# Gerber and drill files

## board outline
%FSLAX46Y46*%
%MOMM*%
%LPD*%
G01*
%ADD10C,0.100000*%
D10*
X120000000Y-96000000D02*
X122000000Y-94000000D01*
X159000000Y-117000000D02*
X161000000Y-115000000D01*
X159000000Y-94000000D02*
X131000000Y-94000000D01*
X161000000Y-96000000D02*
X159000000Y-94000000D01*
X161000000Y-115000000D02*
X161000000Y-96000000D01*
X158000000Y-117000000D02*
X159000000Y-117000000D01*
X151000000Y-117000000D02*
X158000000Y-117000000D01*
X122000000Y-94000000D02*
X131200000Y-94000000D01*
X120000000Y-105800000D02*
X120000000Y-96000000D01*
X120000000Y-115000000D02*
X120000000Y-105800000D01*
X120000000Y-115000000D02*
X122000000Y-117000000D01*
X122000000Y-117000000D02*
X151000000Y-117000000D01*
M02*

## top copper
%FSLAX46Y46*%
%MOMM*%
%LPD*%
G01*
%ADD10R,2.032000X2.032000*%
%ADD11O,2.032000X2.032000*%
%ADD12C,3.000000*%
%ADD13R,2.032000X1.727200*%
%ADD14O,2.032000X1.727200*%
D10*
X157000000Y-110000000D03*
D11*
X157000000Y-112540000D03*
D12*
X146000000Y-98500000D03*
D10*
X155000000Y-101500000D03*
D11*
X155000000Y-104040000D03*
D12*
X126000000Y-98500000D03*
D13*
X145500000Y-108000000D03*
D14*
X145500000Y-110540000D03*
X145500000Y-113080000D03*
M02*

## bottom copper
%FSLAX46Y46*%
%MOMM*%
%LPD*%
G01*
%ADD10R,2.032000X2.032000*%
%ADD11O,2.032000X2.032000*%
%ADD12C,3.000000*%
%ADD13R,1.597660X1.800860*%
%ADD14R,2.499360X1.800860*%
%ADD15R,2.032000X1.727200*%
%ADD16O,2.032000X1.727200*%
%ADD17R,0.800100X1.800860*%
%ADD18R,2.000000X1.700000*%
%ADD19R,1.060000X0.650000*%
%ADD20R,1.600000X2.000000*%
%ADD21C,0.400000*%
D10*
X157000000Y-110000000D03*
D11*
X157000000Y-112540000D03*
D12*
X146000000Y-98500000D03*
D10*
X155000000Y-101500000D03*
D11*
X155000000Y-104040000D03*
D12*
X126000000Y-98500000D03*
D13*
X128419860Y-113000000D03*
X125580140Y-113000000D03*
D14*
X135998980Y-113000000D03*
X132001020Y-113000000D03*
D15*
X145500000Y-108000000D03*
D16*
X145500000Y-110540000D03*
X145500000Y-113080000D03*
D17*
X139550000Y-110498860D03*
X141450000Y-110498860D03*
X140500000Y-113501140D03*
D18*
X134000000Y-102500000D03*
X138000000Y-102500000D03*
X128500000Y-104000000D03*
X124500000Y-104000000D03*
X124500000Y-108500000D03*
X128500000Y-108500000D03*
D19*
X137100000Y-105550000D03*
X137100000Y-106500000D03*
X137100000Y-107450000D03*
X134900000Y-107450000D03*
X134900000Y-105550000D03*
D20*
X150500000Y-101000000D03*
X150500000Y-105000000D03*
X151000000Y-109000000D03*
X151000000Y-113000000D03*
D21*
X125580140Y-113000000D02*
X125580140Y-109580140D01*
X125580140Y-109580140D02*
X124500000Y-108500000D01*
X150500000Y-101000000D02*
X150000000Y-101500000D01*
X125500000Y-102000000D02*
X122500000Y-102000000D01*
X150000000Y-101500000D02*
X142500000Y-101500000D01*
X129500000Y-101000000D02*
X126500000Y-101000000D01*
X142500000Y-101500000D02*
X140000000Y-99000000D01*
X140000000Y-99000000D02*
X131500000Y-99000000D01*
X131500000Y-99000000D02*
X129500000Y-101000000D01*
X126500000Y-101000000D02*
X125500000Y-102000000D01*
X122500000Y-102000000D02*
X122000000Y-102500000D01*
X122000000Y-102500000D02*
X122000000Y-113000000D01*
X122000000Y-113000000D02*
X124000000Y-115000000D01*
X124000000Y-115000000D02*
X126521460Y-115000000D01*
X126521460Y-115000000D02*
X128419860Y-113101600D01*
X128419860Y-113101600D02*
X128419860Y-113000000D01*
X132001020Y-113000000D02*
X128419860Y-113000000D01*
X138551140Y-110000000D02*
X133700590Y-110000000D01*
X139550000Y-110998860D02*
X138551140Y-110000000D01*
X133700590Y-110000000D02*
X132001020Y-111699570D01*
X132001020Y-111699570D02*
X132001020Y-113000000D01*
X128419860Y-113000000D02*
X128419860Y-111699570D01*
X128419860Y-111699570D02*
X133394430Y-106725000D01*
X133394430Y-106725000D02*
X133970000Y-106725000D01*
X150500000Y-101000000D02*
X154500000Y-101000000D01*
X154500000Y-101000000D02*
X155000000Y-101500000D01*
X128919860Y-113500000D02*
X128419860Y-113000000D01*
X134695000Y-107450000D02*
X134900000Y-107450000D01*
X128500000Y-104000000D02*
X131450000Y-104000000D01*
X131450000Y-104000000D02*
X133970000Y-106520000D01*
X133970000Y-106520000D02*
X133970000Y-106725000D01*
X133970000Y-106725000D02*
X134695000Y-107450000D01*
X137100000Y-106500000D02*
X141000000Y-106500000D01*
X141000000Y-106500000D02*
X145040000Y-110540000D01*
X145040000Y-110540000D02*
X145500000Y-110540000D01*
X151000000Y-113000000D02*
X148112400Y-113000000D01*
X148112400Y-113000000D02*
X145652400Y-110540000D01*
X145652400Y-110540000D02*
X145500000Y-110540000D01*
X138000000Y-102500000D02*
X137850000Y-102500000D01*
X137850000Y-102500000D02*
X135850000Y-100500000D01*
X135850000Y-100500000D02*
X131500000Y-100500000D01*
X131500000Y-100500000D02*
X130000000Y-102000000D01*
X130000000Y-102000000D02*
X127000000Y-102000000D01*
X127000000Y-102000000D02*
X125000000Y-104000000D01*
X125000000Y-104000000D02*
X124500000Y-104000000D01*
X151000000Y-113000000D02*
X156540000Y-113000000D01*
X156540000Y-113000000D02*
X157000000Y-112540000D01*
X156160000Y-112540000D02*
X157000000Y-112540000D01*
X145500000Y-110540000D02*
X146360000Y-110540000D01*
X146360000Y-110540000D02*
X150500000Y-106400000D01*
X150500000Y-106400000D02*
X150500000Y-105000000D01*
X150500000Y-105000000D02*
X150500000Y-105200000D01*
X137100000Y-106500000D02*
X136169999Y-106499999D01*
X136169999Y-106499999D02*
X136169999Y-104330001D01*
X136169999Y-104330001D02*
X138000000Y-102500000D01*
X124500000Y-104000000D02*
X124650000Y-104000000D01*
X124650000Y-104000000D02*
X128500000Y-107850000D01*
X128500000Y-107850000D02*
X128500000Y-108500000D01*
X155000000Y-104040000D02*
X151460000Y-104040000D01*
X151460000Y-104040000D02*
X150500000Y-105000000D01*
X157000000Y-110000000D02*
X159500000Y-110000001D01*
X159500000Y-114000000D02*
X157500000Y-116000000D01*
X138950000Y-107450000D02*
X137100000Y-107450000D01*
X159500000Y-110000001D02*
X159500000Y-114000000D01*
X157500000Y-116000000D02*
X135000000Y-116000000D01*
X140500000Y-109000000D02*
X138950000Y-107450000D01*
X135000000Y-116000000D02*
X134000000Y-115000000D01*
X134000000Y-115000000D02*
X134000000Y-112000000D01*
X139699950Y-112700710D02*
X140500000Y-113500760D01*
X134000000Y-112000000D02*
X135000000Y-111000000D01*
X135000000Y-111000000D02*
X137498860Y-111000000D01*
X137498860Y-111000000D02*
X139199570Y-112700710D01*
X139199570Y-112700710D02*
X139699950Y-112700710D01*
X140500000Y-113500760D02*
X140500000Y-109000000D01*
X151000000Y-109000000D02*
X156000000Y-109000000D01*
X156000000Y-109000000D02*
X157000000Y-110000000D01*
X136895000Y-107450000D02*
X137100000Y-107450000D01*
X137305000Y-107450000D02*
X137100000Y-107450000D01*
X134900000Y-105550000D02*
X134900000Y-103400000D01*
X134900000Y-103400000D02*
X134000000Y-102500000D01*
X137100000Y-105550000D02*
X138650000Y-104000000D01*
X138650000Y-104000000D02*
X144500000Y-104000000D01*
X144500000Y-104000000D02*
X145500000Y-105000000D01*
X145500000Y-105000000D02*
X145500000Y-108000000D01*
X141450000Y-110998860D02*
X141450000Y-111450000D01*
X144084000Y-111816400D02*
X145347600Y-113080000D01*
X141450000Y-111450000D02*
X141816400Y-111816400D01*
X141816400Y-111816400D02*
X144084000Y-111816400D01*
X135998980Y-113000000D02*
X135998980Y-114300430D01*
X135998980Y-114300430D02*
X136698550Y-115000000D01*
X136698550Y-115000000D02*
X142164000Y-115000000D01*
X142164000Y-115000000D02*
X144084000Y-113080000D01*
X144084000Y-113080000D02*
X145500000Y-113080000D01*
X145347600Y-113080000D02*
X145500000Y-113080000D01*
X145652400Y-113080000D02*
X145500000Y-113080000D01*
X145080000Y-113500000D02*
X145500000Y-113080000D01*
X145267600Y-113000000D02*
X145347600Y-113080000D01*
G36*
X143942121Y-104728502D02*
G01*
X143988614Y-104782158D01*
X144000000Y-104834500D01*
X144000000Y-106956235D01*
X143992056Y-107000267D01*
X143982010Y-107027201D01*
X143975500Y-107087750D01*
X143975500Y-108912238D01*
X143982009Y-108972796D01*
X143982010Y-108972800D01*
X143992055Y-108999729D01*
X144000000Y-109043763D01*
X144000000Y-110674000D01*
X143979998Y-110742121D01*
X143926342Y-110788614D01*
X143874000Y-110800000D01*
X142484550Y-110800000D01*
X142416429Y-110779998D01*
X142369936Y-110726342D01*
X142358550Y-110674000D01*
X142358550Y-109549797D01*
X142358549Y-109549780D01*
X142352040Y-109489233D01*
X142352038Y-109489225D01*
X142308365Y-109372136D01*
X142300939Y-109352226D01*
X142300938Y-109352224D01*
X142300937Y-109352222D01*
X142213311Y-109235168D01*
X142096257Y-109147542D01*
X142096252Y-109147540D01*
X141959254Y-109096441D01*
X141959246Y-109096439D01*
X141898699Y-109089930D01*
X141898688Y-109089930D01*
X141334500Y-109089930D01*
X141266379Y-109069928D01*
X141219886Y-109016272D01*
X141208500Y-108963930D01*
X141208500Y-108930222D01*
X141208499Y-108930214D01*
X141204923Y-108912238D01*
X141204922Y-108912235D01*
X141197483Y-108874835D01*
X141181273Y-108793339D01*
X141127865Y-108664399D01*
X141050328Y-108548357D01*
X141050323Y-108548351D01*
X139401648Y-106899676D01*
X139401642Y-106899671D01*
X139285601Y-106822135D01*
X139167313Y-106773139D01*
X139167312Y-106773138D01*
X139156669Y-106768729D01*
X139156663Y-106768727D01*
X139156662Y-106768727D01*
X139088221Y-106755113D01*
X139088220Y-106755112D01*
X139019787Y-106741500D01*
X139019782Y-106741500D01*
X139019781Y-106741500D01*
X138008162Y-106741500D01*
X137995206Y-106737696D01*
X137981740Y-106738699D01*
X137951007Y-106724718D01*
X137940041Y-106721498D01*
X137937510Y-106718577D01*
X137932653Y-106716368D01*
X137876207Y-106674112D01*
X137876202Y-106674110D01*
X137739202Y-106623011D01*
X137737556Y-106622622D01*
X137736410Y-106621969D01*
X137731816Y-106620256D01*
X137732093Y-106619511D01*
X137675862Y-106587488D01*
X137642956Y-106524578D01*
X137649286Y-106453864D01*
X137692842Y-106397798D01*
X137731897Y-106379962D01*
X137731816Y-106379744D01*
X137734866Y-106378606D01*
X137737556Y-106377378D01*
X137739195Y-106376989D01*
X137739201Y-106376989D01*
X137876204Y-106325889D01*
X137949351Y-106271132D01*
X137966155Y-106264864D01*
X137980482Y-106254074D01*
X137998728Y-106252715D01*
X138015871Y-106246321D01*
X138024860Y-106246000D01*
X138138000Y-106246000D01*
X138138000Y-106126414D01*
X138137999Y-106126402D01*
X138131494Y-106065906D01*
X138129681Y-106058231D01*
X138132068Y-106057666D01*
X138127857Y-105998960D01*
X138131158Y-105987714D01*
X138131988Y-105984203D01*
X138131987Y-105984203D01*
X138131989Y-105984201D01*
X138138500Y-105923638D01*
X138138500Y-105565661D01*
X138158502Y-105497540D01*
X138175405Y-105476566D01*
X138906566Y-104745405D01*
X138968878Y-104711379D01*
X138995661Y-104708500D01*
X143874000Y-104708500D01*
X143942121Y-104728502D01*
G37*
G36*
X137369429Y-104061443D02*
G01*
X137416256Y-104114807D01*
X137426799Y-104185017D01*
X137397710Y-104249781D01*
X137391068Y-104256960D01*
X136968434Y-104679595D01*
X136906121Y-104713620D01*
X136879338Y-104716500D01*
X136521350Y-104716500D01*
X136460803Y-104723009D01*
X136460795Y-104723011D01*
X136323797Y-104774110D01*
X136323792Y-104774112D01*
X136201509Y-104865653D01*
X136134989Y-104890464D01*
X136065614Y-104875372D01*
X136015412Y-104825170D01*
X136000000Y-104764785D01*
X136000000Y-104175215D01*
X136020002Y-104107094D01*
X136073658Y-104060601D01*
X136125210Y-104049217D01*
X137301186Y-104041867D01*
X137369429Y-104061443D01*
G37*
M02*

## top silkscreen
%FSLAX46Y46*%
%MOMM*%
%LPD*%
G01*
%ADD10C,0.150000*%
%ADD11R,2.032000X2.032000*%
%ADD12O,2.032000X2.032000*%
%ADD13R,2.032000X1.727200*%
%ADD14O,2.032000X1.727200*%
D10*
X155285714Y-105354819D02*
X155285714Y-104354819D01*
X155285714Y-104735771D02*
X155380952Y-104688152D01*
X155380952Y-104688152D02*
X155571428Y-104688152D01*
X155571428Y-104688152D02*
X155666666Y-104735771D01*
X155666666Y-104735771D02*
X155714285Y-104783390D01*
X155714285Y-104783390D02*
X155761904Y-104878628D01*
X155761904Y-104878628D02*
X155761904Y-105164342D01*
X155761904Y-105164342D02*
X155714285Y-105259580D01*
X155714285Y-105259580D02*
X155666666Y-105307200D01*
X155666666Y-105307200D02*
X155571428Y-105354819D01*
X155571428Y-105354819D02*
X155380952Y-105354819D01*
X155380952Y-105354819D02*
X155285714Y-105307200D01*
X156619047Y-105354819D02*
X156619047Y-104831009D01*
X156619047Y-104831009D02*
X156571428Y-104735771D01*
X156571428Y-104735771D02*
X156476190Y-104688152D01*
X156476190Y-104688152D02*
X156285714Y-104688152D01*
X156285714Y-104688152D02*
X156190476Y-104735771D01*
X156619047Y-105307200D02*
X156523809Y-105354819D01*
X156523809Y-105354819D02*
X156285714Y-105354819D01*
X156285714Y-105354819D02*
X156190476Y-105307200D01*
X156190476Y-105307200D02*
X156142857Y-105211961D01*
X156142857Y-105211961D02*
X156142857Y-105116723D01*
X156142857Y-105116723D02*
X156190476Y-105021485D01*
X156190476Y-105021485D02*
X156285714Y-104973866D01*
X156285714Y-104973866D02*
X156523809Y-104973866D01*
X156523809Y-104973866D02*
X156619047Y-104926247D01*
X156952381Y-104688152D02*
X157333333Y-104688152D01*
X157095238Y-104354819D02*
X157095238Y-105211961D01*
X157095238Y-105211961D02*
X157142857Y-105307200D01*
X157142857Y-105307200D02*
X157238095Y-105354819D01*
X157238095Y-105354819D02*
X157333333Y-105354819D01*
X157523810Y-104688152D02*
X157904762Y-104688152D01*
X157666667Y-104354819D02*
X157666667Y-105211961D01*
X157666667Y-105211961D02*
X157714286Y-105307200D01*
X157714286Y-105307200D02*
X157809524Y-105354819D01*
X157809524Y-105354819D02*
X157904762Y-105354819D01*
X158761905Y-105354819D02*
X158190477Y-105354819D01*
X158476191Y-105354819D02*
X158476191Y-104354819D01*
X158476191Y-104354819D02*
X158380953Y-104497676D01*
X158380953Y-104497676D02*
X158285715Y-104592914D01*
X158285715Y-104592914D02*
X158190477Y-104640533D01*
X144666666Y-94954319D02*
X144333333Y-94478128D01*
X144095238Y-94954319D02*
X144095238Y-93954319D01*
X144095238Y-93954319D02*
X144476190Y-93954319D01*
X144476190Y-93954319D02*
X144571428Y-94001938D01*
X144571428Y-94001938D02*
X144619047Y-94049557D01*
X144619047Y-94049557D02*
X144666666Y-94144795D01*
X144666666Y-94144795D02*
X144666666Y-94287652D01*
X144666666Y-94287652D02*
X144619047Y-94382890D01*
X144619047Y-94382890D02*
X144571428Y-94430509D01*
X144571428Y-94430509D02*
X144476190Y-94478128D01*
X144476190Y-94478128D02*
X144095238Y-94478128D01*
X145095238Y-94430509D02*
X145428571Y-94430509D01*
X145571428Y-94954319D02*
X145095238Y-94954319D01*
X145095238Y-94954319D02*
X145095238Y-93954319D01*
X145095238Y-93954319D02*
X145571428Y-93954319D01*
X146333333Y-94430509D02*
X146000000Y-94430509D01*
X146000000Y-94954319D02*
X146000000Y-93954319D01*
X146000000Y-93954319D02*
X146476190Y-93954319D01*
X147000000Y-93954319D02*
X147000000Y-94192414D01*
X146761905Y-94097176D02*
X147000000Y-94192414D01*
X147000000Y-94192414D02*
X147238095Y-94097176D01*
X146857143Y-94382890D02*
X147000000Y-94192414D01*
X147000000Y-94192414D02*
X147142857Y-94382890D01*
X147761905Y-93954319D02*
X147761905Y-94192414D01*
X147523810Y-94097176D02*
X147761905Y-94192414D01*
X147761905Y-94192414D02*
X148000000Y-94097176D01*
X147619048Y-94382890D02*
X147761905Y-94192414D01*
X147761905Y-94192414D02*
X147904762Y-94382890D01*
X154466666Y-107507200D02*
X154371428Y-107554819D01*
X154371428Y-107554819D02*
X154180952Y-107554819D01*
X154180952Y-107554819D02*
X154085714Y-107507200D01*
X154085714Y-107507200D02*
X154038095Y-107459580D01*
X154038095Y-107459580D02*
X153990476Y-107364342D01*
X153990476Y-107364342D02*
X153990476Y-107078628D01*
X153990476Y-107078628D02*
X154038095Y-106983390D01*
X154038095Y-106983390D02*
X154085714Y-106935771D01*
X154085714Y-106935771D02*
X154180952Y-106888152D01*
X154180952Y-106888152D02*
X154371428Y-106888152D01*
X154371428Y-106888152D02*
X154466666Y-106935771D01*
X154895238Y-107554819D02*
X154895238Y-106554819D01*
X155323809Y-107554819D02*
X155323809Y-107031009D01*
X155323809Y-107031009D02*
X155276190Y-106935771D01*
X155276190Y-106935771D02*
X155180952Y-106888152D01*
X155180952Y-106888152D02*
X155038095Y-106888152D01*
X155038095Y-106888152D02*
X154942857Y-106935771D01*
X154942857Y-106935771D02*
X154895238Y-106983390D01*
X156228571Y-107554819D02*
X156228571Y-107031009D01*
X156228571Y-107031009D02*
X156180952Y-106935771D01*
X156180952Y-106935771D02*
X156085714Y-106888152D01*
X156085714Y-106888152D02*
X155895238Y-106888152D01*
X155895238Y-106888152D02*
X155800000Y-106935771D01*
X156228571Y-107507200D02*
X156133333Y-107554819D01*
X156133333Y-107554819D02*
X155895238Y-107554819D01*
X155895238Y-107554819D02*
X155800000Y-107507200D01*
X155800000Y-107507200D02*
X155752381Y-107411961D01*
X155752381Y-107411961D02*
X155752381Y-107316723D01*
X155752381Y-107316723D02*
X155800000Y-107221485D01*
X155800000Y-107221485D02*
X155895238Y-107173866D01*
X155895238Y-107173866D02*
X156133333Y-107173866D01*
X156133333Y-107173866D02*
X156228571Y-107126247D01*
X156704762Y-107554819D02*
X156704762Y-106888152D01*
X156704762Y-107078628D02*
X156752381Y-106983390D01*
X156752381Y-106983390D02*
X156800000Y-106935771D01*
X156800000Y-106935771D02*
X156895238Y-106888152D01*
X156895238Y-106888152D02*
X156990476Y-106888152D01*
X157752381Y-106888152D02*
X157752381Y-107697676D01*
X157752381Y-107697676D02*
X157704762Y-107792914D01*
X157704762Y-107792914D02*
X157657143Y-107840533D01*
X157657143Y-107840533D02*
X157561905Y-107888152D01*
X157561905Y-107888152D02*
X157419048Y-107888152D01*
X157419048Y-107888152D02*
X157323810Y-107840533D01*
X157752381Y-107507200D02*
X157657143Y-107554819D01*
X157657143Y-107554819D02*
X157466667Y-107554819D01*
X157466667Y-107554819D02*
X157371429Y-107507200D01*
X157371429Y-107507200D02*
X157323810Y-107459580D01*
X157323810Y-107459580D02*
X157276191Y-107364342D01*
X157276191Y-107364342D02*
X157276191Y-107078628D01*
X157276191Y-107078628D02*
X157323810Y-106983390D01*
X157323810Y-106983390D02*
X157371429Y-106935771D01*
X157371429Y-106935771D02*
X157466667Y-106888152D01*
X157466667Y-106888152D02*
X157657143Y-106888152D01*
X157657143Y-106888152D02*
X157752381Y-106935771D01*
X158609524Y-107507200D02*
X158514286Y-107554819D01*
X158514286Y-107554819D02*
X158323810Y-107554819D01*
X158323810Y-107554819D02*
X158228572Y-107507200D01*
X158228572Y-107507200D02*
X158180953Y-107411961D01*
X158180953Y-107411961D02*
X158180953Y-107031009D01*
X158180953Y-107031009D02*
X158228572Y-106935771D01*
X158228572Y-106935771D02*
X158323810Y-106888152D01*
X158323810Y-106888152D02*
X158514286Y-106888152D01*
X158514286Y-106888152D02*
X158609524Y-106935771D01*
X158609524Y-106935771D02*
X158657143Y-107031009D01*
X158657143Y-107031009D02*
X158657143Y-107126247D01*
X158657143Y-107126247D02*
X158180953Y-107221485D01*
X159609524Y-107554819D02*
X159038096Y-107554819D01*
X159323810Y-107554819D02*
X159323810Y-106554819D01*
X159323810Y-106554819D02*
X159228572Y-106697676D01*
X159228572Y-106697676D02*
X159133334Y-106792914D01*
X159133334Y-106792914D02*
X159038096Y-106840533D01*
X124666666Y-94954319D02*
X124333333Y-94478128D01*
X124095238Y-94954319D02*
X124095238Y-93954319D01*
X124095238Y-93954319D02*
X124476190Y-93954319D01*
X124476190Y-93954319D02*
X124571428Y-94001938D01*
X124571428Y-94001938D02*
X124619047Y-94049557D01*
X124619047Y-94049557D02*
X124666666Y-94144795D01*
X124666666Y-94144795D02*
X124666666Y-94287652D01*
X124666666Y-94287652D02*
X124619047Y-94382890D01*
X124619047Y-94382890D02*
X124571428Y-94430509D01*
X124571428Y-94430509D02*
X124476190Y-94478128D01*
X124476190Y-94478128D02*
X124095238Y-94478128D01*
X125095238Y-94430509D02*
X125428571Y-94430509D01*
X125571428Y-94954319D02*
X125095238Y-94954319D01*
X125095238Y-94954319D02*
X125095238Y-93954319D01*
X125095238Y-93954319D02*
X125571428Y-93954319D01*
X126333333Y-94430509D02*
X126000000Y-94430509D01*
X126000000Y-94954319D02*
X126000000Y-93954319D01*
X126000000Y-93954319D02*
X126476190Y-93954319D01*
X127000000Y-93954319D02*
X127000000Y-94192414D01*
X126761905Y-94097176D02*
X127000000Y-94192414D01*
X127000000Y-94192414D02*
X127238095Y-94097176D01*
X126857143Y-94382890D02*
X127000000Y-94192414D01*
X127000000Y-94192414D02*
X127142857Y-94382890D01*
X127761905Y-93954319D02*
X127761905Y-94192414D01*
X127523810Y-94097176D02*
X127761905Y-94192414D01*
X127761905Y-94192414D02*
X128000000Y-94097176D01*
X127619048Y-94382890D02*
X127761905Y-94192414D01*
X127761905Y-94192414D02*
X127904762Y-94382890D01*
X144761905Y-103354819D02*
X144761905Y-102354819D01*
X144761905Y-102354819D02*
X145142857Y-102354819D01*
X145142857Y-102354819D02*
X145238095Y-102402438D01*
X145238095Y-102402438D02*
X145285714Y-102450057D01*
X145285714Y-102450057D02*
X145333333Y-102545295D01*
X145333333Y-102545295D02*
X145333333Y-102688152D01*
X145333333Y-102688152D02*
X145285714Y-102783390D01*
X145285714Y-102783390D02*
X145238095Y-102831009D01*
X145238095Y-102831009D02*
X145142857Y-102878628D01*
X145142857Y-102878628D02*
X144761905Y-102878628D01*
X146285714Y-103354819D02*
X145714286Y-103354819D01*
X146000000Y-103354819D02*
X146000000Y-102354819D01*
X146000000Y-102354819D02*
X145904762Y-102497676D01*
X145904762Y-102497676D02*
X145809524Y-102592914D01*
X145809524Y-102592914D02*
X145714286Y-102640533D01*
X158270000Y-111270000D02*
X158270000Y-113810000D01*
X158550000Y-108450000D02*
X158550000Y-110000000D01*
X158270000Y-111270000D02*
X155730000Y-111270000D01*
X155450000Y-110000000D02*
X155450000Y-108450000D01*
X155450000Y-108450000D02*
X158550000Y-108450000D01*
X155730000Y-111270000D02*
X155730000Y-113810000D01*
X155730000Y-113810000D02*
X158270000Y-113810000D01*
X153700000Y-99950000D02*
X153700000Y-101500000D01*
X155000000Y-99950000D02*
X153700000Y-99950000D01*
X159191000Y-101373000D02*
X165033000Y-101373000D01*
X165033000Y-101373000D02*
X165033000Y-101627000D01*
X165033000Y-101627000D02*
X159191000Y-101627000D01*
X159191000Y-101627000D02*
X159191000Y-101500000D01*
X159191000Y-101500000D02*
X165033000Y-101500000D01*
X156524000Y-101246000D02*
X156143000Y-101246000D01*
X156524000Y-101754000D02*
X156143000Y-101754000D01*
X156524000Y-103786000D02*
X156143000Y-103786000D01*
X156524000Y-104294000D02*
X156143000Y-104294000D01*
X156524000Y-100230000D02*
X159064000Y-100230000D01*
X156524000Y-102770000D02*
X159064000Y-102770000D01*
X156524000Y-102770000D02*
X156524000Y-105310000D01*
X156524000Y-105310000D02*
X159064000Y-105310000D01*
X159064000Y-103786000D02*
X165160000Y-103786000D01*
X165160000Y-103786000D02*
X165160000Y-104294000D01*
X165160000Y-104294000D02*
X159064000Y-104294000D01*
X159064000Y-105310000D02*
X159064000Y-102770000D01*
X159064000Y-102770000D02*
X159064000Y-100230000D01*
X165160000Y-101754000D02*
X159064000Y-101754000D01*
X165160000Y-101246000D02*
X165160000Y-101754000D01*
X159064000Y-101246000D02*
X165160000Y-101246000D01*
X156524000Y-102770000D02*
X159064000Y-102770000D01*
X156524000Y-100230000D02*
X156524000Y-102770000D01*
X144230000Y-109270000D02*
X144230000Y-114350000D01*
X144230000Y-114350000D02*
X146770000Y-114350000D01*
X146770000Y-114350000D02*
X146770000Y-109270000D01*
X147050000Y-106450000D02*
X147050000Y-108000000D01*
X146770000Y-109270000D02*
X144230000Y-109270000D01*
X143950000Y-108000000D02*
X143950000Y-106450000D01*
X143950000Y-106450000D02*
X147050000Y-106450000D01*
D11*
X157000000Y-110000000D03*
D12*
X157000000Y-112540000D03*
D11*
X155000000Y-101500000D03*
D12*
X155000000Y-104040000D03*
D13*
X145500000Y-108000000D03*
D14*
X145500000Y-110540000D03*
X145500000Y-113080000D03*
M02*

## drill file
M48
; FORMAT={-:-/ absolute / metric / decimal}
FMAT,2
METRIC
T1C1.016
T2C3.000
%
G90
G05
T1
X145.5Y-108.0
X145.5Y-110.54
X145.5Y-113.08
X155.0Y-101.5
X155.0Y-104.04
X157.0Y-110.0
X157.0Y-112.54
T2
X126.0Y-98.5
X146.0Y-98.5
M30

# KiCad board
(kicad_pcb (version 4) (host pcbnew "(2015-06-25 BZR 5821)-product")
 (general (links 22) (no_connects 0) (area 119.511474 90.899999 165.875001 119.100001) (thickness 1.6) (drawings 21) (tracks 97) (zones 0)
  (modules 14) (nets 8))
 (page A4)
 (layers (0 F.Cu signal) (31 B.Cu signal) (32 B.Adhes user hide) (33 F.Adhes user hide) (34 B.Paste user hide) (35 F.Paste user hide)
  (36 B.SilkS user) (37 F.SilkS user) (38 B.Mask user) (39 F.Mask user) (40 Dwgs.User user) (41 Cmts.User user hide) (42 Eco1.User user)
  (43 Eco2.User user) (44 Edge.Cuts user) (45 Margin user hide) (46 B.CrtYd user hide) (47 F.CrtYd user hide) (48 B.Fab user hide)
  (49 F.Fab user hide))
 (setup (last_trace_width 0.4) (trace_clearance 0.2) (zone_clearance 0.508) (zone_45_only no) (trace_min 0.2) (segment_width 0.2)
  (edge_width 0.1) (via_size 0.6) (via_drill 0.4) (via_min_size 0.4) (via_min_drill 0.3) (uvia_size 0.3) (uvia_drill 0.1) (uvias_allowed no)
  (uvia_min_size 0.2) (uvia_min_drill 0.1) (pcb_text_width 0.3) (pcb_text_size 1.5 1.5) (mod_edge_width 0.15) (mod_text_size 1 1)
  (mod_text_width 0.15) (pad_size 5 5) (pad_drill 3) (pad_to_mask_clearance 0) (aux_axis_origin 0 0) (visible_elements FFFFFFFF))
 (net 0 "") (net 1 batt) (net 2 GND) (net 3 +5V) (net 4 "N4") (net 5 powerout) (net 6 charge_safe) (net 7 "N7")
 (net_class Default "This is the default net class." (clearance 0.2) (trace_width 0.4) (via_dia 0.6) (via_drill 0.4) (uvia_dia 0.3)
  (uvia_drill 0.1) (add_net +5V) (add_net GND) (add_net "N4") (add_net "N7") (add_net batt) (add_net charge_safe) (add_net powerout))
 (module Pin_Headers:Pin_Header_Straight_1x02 (layer F.Cu) (at 157 110)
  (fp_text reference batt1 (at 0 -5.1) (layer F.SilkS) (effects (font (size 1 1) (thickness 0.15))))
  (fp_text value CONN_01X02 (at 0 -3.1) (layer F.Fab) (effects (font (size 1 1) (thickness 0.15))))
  (fp_line (start 1.27 1.27) (end 1.27 3.81) (layer F.SilkS) (width 0.15))
  (fp_line (start 1.55 -1.55) (end 1.55 0) (layer F.SilkS) (width 0.15))
  (fp_line (start 1.27 1.27) (end -1.27 1.27) (layer F.SilkS) (width 0.15))
  (fp_line (start -1.55 0) (end -1.55 -1.55) (layer F.SilkS) (width 0.15))
  (fp_line (start -1.55 -1.55) (end 1.55 -1.55) (layer F.SilkS) (width 0.15))
  (fp_line (start -1.27 1.27) (end -1.27 3.81) (layer F.SilkS) (width 0.15))
  (fp_line (start -1.27 3.81) (end 1.27 3.81) (layer F.SilkS) (width 0.15))
  (pad 1 thru_hole rect (at 0 0) (size 2.032 2.032) (drill 1.016) (layers *.Cu *.Mask F.SilkS) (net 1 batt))
  (pad 2 thru_hole oval (at 0 2.54) (size 2.032 2.032) (drill 1.016) (layers *.Cu *.Mask F.SilkS) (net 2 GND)))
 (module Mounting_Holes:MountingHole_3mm (layer F.Cu) (at 146 98.5)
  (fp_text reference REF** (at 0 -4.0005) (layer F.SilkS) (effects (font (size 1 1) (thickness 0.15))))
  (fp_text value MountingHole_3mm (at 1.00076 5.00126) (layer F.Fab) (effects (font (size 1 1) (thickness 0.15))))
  (pad 1 thru_hole circle (at 0 0) (size 3 3) (drill 3) (layers)))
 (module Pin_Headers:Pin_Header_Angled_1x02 (layer F.Cu) (at 155 101.5)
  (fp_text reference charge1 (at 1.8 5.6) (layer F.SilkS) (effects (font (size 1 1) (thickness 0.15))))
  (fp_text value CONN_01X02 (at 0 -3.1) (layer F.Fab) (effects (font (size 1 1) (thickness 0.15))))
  (fp_line (start -1.3 -1.55) (end -1.3 0) (layer F.SilkS) (width 0.15))
  (fp_line (start 0 -1.55) (end -1.3 -1.55) (layer F.SilkS) (width 0.15))
  (fp_line (start 4.191 -0.127) (end 10.033 -0.127) (layer F.SilkS) (width 0.15))
  (fp_line (start 10.033 -0.127) (end 10.033 0.127) (layer F.SilkS) (width 0.15))
  (fp_line (start 10.033 0.127) (end 4.191 0.127) (layer F.SilkS) (width 0.15))
  (fp_line (start 4.191 0.127) (end 4.191 0) (layer F.SilkS) (width 0.15))
  (fp_line (start 4.191 0) (end 10.033 0) (layer F.SilkS) (width 0.15))
  (fp_line (start 1.524 -0.254) (end 1.143 -0.254) (layer F.SilkS) (width 0.15))
  (fp_line (start 1.524 0.254) (end 1.143 0.254) (layer F.SilkS) (width 0.15))
  (fp_line (start 1.524 2.286) (end 1.143 2.286) (layer F.SilkS) (width 0.15))
  (fp_line (start 1.524 2.794) (end 1.143 2.794) (layer F.SilkS) (width 0.15))
  (fp_line (start 1.524 -1.27) (end 4.064 -1.27) (layer F.SilkS) (width 0.15))
  (fp_line (start 1.524 1.27) (end 4.064 1.27) (layer F.SilkS) (width 0.15))
  (fp_line (start 1.524 1.27) (end 1.524 3.81) (layer F.SilkS) (width 0.15))
  (fp_line (start 1.524 3.81) (end 4.064 3.81) (layer F.SilkS) (width 0.15))
  (fp_line (start 4.064 2.286) (end 10.16 2.286) (layer F.SilkS) (width 0.15))
  (fp_line (start 10.16 2.286) (end 10.16 2.794) (layer F.SilkS) (width 0.15))
  (fp_line (start 10.16 2.794) (end 4.064 2.794) (layer F.SilkS) (width 0.15))
  (fp_line (start 4.064 3.81) (end 4.064 1.27) (layer F.SilkS) (width 0.15))
  (fp_line (start 4.064 1.27) (end 4.064 -1.27) (layer F.SilkS) (width 0.15))
  (fp_line (start 10.16 0.254) (end 4.064 0.254) (layer F.SilkS) (width 0.15))
  (fp_line (start 10.16 -0.254) (end 10.16 0.254) (layer F.SilkS) (width 0.15))
  (fp_line (start 4.064 -0.254) (end 10.16 -0.254) (layer F.SilkS) (width 0.15))
  (fp_line (start 1.524 1.27) (end 4.064 1.27) (layer F.SilkS) (width 0.15))
  (fp_line (start 1.524 -1.27) (end 1.524 1.27) (layer F.SilkS) (width 0.15))
  (pad 1 thru_hole rect (at 0 0) (size 2.032 2.032) (drill 1.016) (layers *.Cu *.Mask F.SilkS) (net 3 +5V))
  (pad 2 thru_hole oval (at 0 2.54) (size 2.032 2.032) (drill 1.016) (layers *.Cu *.Mask F.SilkS) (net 2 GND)))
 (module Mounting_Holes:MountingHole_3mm (layer F.Cu) (at 126 98.5)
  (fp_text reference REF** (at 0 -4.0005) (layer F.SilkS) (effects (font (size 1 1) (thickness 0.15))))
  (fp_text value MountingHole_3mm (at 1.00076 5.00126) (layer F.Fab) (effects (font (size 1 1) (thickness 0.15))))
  (pad 1 thru_hole circle (at 0 0) (size 3 3) (drill 3) (layers)))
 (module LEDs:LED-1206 (layer B.Cu) (at 127 113)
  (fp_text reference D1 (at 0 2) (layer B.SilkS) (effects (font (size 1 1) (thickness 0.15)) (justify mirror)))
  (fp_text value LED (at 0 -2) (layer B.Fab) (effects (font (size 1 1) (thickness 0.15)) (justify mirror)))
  (pad 2 smd rect (at 1.41986 0 180) (size 1.59766 1.80086) (layers B.Cu B.Paste B.Mask) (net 3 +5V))
  (pad 1 smd rect (at -1.41986 0 180) (size 1.59766 1.80086) (layers B.Cu B.Paste B.Mask) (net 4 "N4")))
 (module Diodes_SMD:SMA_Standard (layer B.Cu) (at 134 113 180)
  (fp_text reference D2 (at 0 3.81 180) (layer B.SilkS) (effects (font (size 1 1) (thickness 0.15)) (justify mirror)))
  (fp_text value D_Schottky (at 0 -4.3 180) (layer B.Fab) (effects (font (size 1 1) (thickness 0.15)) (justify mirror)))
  (pad 1 smd rect (at -1.99898 0 180) (size 2.49936 1.80086) (layers B.Cu B.Paste B.Mask) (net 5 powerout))
  (pad 2 smd rect (at 1.99898 0 180) (size 2.49936 1.80086) (layers B.Cu B.Paste B.Mask) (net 3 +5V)))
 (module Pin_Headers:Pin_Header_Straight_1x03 (layer F.Cu) (at 145.5 108)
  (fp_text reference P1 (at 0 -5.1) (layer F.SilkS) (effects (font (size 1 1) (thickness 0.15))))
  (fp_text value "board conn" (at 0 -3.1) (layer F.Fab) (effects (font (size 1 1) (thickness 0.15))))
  (fp_line (start -1.27 1.27) (end -1.27 6.35) (layer F.SilkS) (width 0.15))
  (fp_line (start -1.27 6.35) (end 1.27 6.35) (layer F.SilkS) (width 0.15))
  (fp_line (start 1.27 6.35) (end 1.27 1.27) (layer F.SilkS) (width 0.15))
  (fp_line (start 1.55 -1.55) (end 1.55 0) (layer F.SilkS) (width 0.15))
  (fp_line (start 1.27 1.27) (end -1.27 1.27) (layer F.SilkS) (width 0.15))
  (fp_line (start -1.55 0) (end -1.55 -1.55) (layer F.SilkS) (width 0.15))
  (fp_line (start -1.55 -1.55) (end 1.55 -1.55) (layer F.SilkS) (width 0.15))
  (pad 1 thru_hole rect (at 0 0) (size 2.032 1.7272) (drill 1.016) (layers *.Cu *.Mask F.SilkS) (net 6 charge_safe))
  (pad 2 thru_hole oval (at 0 2.54) (size 2.032 1.7272) (drill 1.016) (layers *.Cu *.Mask F.SilkS) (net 2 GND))
  (pad 3 thru_hole oval (at 0 5.08) (size 2.032 1.7272) (drill 1.016) (layers *.Cu *.Mask F.SilkS) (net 5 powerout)))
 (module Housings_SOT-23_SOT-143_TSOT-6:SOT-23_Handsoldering (layer B.Cu) (at 140.5 112)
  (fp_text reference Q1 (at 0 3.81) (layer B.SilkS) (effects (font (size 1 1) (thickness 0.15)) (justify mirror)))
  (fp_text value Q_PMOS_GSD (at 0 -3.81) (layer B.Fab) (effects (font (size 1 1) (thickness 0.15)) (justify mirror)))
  (pad 1 smd rect (at -0.95 -1.50114) (size 0.8001 1.80086) (layers B.Cu B.Paste B.Mask) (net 3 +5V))
  (pad 2 smd rect (at 0.95 -1.50114) (size 0.8001 1.80086) (layers B.Cu B.Paste B.Mask) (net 5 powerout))
  (pad 3 smd rect (at 0 1.50114) (size 0.8001 1.80086) (layers B.Cu B.Paste B.Mask) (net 1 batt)))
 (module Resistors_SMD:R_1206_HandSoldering (layer B.Cu) (at 136 102.5)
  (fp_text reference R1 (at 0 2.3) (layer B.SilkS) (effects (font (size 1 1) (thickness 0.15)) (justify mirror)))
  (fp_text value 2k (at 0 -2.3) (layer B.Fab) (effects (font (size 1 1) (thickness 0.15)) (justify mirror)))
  (pad 1 smd rect (at -2 0) (size 2 1.7) (layers B.Cu B.Paste B.Mask) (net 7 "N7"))
  (pad 2 smd rect (at 2 0) (size 2 1.7) (layers B.Cu B.Paste B.Mask) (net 2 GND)))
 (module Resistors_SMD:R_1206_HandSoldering (layer B.Cu) (at 126.5 104 180)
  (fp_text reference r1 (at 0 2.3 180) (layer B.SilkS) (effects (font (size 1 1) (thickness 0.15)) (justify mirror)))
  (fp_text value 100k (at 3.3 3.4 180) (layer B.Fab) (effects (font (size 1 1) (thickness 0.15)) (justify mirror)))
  (pad 1 smd rect (at -2 0 180) (size 2 1.7) (layers B.Cu B.Paste B.Mask) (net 3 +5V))
  (pad 2 smd rect (at 2 0 180) (size 2 1.7) (layers B.Cu B.Paste B.Mask) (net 2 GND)))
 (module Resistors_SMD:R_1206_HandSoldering (layer B.Cu) (at 126.5 108.5)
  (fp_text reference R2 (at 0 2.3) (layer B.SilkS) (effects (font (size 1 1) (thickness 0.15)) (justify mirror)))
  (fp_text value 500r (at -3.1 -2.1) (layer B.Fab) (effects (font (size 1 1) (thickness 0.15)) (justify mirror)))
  (pad 1 smd rect (at -2 0) (size 2 1.7) (layers B.Cu B.Paste B.Mask) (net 4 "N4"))
  (pad 2 smd rect (at 2 0) (size 2 1.7) (layers B.Cu B.Paste B.Mask) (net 2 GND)))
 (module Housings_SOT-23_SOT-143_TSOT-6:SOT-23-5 (layer B.Cu) (at 136 106.5 180)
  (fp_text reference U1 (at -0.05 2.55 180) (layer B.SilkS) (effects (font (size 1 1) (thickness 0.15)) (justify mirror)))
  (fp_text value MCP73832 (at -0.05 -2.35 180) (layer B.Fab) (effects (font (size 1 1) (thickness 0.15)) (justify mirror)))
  (pad 1 smd rect (at -1.1 0.95 180) (size 1.06 0.65) (layers B.Cu B.Paste B.Mask) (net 6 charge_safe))
  (pad 2 smd rect (at -1.1 0 180) (size 1.06 0.65) (layers B.Cu B.Paste B.Mask) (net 2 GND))
  (pad 3 smd rect (at -1.1 -0.95 180) (size 1.06 0.65) (layers B.Cu B.Paste B.Mask) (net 1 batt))
  (pad 4 smd rect (at 1.1 -0.95 180) (size 1.06 0.65) (layers B.Cu B.Paste B.Mask) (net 3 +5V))
  (pad 5 smd rect (at 1.1 0.95 180) (size 1.06 0.65) (layers B.Cu B.Paste B.Mask) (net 7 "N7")))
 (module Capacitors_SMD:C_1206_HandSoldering (layer B.Cu) (at 150.5 103 270)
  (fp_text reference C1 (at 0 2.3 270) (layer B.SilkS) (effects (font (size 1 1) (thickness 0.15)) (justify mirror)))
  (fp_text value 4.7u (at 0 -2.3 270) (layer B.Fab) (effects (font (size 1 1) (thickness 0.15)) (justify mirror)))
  (pad 1 smd rect (at -2 0 270) (size 2 1.6) (layers B.Cu B.Paste B.Mask) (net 3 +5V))
  (pad 2 smd rect (at 2 0 270) (size 2 1.6) (layers B.Cu B.Paste B.Mask) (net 2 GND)))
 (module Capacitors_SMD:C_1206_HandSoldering (layer B.Cu) (at 151 111 270)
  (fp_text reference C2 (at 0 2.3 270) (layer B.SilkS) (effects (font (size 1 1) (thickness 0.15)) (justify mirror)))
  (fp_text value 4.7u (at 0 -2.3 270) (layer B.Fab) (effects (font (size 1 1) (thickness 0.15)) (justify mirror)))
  (pad 1 smd rect (at -2 0 270) (size 2 1.6) (layers B.Cu B.Paste B.Mask) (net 1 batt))
  (pad 2 smd rect (at 2 0 270) (size 2 1.6) (layers B.Cu B.Paste B.Mask) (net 2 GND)))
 (gr_line (start 120 96) (end 122 94) (layer Edge.Cuts) (width 0.1))
 (gr_line (start 159 117) (end 161 115) (angle 90) (layer Edge.Cuts) (width 0.1))
 (gr_line (start 159 94) (end 131 94) (layer Edge.Cuts) (width 0.1))
 (gr_line (start 161 96) (end 159 94) (layer Edge.Cuts) (width 0.1))
 (gr_line (start 161 115) (end 161 96) (layer Edge.Cuts) (width 0.1))
 (gr_line (start 158 117) (end 159 117) (layer Edge.Cuts) (width 0.1))
 (gr_line (start 151 117) (end 158 117) (layer Edge.Cuts) (width 0.1))
 (gr_line (start 122 94) (end 131.2 94) (layer Edge.Cuts) (width 0.1))
 (gr_line (start 120 105.8) (end 120 96) (layer Edge.Cuts) (width 0.1))
 (gr_line (start 120 115) (end 120 105.8) (angle 90) (layer Edge.Cuts) (width 0.1))
 (gr_line (start 120 115) (end 122 117) (layer Edge.Cuts) (width 0.1))
 (gr_line (start 122 117) (end 151 117) (layer Edge.Cuts) (width 0.1))
 (segment (start 125.58014 113) (end 125.58014 109.58014) (width 0.4) (layer B.Cu) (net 4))
 (segment (start 125.58014 109.58014) (end 124.5 108.5) (width 0.4) (layer B.Cu) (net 4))
 (segment (start 150.5 101) (end 150 101.5) (width 0.4) (layer B.Cu) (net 3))
 (segment (start 125.5 102) (end 122.5 102) (width 0.4) (layer B.Cu) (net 3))
 (segment (start 150 101.5) (end 142.5 101.5) (width 0.4) (layer B.Cu) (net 3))
 (segment (start 129.5 101) (end 126.5 101) (width 0.4) (layer B.Cu) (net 3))
 (segment (start 142.5 101.5) (end 140 99) (width 0.4) (layer B.Cu) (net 3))
 (segment (start 140 99) (end 131.5 99) (width 0.4) (layer B.Cu) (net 3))
 (segment (start 131.5 99) (end 129.5 101) (width 0.4) (layer B.Cu) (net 3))
 (segment (start 126.5 101) (end 125.5 102) (width 0.4) (layer B.Cu) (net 3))
 (segment (start 122.5 102) (end 122 102.5) (width 0.4) (layer B.Cu) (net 3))
 (segment (start 122 102.5) (end 122 113) (width 0.4) (layer B.Cu) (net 3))
 (segment (start 122 113) (end 124 115) (width 0.4) (layer B.Cu) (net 3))
 (segment (start 124 115) (end 126.52146 115) (width 0.4) (layer B.Cu) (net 3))
 (segment (start 126.52146 115) (end 128.41986 113.1016) (width 0.4) (layer B.Cu) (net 3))
 (segment (start 128.41986 113.1016) (end 128.41986 113) (width 0.4) (layer B.Cu) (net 3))
 (segment (start 132.00102 113) (end 128.41986 113) (width 0.4) (layer B.Cu) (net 3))
 (segment (start 138.55114 110) (end 133.70059 110) (width 0.4) (layer B.Cu) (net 3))
 (segment (start 139.55 110.99886) (end 138.55114 110) (width 0.4) (layer B.Cu) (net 3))
 (segment (start 133.70059 110) (end 132.00102 111.69957) (width 0.4) (layer B.Cu) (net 3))
 (segment (start 132.00102 111.69957) (end 132.00102 113) (width 0.4) (layer B.Cu) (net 3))
 (segment (start 128.41986 113) (end 128.41986 111.69957) (width 0.4) (layer B.Cu) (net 3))
 (segment (start 128.41986 111.69957) (end 133.39443 106.725) (width 0.4) (layer B.Cu) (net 3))
 (segment (start 133.39443 106.725) (end 133.97 106.725) (width 0.4) (layer B.Cu) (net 3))
 (segment (start 150.5 101) (end 154.5 101) (width 0.4) (layer B.Cu) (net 3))
 (segment (start 154.5 101) (end 155 101.5) (width 0.4) (layer B.Cu) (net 3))
 (segment (start 128.91986 113.5) (end 128.41986 113) (width 0.4) (layer B.Cu) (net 3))
 (segment (start 134.695 107.45) (end 134.9 107.45) (width 0.4) (layer B.Cu) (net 3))
 (segment (start 128.5 104) (end 131.45 104) (width 0.4) (layer B.Cu) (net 3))
 (segment (start 131.45 104) (end 133.97 106.52) (width 0.4) (layer B.Cu) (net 3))
 (segment (start 133.97 106.52) (end 133.97 106.725) (width 0.4) (layer B.Cu) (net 3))
 (segment (start 133.97 106.725) (end 134.695 107.45) (width 0.4) (layer B.Cu) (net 3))
 (segment (start 137.1 106.5) (end 141 106.5) (width 0.4) (layer B.Cu) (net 2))
 (segment (start 141 106.5) (end 145.04 110.54) (width 0.4) (layer B.Cu) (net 2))
 (segment (start 145.04 110.54) (end 145.5 110.54) (width 0.4) (layer B.Cu) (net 2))
 (segment (start 151 113) (end 148.1124 113) (width 0.4) (layer B.Cu) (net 2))
 (segment (start 148.1124 113) (end 145.6524 110.54) (width 0.4) (layer B.Cu) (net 2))
 (segment (start 145.6524 110.54) (end 145.5 110.54) (width 0.4) (layer B.Cu) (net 2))
 (segment (start 138 102.5) (end 137.85 102.5) (width 0.4) (layer B.Cu) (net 2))
 (segment (start 137.85 102.5) (end 135.85 100.5) (width 0.4) (layer B.Cu) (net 2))
 (segment (start 135.85 100.5) (end 131.5 100.5) (width 0.4) (layer B.Cu) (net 2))
 (segment (start 131.5 100.5) (end 130 102) (width 0.4) (layer B.Cu) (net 2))
 (segment (start 130 102) (end 127 102) (width 0.4) (layer B.Cu) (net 2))
 (segment (start 127 102) (end 125 104) (width 0.4) (layer B.Cu) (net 2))
 (segment (start 125 104) (end 124.5 104) (width 0.4) (layer B.Cu) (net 2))
 (segment (start 151 113) (end 156.54 113) (width 0.4) (layer B.Cu) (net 2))
 (segment (start 156.54 113) (end 157 112.54) (width 0.4) (layer B.Cu) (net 2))
 (segment (start 156.16 112.54) (end 157 112.54) (width 0.4) (layer B.Cu) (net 2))
 (segment (start 145.5 110.54) (end 146.36 110.54) (width 0.4) (layer B.Cu) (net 2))
 (segment (start 146.36 110.54) (end 150.5 106.4) (width 0.4) (layer B.Cu) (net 2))
 (segment (start 150.5 106.4) (end 150.5 105) (width 0.4) (layer B.Cu) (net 2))
 (segment (start 150.5 105) (end 150.5 105.2) (width 0.4) (layer B.Cu) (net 2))
 (segment (start 137.1 106.5) (end 136.169999 106.499999) (width 0.4) (layer B.Cu) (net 2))
 (segment (start 136.169999 106.499999) (end 136.169999 104.330001) (width 0.4) (layer B.Cu) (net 2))
 (segment (start 136.169999 104.330001) (end 138 102.5) (width 0.4) (layer B.Cu) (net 2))
 (segment (start 124.5 104) (end 124.65 104) (width 0.4) (layer B.Cu) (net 2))
 (segment (start 124.65 104) (end 128.5 107.85) (width 0.4) (layer B.Cu) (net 2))
 (segment (start 128.5 107.85) (end 128.5 108.5) (width 0.4) (layer B.Cu) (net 2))
 (segment (start 155 104.04) (end 151.46 104.04) (width 0.4) (layer B.Cu) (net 2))
 (segment (start 151.46 104.04) (end 150.5 105) (width 0.4) (layer B.Cu) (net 2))
 (segment (start 157 110) (end 159.5 110.000001) (width 0.4) (layer B.Cu) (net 1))
 (segment (start 159.5 114) (end 157.5 116) (width 0.4) (layer B.Cu) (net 1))
 (segment (start 138.95 107.45) (end 137.1 107.45) (width 0.4) (layer B.Cu) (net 1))
 (segment (start 159.5 110.000001) (end 159.5 114) (width 0.4) (layer B.Cu) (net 1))
 (segment (start 157.5 116) (end 135 116) (width 0.4) (layer B.Cu) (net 1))
 (segment (start 140.5 109) (end 138.95 107.45) (width 0.4) (layer B.Cu) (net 1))
 (segment (start 135 116) (end 134 115) (width 0.4) (layer B.Cu) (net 1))
 (segment (start 134 115) (end 134 112) (width 0.4) (layer B.Cu) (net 1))
 (segment (start 139.69995 112.70071) (end 140.5 113.50076) (width 0.4) (layer B.Cu) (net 1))
 (segment (start 134 112) (end 135 111) (width 0.4) (layer B.Cu) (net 1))
 (segment (start 135 111) (end 137.49886 111) (width 0.4) (layer B.Cu) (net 1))
 (segment (start 137.49886 111) (end 139.19957 112.70071) (width 0.4) (layer B.Cu) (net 1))
 (segment (start 139.19957 112.70071) (end 139.69995 112.70071) (width 0.4) (layer B.Cu) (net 1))
 (segment (start 140.5 113.50076) (end 140.5 109) (width 0.4) (layer B.Cu) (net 1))
 (segment (start 151 109) (end 156 109) (width 0.4) (layer B.Cu) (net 1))
 (segment (start 156 109) (end 157 110) (width 0.4) (layer B.Cu) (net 1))
 (segment (start 136.895 107.45) (end 137.1 107.45) (width 0.4) (layer B.Cu) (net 1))
 (segment (start 137.305 107.45) (end 137.1 107.45) (width 0.4) (layer B.Cu) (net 1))
 (segment (start 134.9 105.55) (end 134.9 103.4) (width 0.4) (layer B.Cu) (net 7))
 (segment (start 134.9 103.4) (end 134 102.5) (width 0.4) (layer B.Cu) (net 7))
 (segment (start 137.1 105.55) (end 138.65 104) (width 0.4) (layer B.Cu) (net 6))
 (segment (start 138.65 104) (end 144.5 104) (width 0.4) (layer B.Cu) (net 6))
 (segment (start 144.5 104) (end 145.5 105) (width 0.4) (layer B.Cu) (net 6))
 (segment (start 145.5 105) (end 145.5 108) (width 0.4) (layer B.Cu) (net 6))
 (segment (start 141.45 110.99886) (end 141.45 111.45) (width 0.4) (layer B.Cu) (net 5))
 (segment (start 144.084 111.8164) (end 145.3476 113.08) (width 0.4) (layer B.Cu) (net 5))
 (segment (start 141.45 111.45) (end 141.8164 111.8164) (width 0.4) (layer B.Cu) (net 5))
 (segment (start 141.8164 111.8164) (end 144.084 111.8164) (width 0.4) (layer B.Cu) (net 5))
 (segment (start 135.99898 113) (end 135.99898 114.30043) (width 0.4) (layer B.Cu) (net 5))
 (segment (start 135.99898 114.30043) (end 136.69855 115) (width 0.4) (layer B.Cu) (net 5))
 (segment (start 136.69855 115) (end 142.164 115) (width 0.4) (layer B.Cu) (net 5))
 (segment (start 142.164 115) (end 144.084 113.08) (width 0.4) (layer B.Cu) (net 5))
 (segment (start 144.084 113.08) (end 145.5 113.08) (width 0.4) (layer B.Cu) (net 5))
 (segment (start 145.3476 113.08) (end 145.5 113.08) (width 0.4) (layer B.Cu) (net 5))
 (segment (start 145.6524 113.08) (end 145.5 113.08) (width 0.4) (layer B.Cu) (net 5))
 (segment (start 145.08 113.5) (end 145.5 113.08) (width 0.4) (layer B.Cu) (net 5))
 (segment (start 145.2676 113) (end 145.3476 113.08) (width 0.4) (layer B.Cu) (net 5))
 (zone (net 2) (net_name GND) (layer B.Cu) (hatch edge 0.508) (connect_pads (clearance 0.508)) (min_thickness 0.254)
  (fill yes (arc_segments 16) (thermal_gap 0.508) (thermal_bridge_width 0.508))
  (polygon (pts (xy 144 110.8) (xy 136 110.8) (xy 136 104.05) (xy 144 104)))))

